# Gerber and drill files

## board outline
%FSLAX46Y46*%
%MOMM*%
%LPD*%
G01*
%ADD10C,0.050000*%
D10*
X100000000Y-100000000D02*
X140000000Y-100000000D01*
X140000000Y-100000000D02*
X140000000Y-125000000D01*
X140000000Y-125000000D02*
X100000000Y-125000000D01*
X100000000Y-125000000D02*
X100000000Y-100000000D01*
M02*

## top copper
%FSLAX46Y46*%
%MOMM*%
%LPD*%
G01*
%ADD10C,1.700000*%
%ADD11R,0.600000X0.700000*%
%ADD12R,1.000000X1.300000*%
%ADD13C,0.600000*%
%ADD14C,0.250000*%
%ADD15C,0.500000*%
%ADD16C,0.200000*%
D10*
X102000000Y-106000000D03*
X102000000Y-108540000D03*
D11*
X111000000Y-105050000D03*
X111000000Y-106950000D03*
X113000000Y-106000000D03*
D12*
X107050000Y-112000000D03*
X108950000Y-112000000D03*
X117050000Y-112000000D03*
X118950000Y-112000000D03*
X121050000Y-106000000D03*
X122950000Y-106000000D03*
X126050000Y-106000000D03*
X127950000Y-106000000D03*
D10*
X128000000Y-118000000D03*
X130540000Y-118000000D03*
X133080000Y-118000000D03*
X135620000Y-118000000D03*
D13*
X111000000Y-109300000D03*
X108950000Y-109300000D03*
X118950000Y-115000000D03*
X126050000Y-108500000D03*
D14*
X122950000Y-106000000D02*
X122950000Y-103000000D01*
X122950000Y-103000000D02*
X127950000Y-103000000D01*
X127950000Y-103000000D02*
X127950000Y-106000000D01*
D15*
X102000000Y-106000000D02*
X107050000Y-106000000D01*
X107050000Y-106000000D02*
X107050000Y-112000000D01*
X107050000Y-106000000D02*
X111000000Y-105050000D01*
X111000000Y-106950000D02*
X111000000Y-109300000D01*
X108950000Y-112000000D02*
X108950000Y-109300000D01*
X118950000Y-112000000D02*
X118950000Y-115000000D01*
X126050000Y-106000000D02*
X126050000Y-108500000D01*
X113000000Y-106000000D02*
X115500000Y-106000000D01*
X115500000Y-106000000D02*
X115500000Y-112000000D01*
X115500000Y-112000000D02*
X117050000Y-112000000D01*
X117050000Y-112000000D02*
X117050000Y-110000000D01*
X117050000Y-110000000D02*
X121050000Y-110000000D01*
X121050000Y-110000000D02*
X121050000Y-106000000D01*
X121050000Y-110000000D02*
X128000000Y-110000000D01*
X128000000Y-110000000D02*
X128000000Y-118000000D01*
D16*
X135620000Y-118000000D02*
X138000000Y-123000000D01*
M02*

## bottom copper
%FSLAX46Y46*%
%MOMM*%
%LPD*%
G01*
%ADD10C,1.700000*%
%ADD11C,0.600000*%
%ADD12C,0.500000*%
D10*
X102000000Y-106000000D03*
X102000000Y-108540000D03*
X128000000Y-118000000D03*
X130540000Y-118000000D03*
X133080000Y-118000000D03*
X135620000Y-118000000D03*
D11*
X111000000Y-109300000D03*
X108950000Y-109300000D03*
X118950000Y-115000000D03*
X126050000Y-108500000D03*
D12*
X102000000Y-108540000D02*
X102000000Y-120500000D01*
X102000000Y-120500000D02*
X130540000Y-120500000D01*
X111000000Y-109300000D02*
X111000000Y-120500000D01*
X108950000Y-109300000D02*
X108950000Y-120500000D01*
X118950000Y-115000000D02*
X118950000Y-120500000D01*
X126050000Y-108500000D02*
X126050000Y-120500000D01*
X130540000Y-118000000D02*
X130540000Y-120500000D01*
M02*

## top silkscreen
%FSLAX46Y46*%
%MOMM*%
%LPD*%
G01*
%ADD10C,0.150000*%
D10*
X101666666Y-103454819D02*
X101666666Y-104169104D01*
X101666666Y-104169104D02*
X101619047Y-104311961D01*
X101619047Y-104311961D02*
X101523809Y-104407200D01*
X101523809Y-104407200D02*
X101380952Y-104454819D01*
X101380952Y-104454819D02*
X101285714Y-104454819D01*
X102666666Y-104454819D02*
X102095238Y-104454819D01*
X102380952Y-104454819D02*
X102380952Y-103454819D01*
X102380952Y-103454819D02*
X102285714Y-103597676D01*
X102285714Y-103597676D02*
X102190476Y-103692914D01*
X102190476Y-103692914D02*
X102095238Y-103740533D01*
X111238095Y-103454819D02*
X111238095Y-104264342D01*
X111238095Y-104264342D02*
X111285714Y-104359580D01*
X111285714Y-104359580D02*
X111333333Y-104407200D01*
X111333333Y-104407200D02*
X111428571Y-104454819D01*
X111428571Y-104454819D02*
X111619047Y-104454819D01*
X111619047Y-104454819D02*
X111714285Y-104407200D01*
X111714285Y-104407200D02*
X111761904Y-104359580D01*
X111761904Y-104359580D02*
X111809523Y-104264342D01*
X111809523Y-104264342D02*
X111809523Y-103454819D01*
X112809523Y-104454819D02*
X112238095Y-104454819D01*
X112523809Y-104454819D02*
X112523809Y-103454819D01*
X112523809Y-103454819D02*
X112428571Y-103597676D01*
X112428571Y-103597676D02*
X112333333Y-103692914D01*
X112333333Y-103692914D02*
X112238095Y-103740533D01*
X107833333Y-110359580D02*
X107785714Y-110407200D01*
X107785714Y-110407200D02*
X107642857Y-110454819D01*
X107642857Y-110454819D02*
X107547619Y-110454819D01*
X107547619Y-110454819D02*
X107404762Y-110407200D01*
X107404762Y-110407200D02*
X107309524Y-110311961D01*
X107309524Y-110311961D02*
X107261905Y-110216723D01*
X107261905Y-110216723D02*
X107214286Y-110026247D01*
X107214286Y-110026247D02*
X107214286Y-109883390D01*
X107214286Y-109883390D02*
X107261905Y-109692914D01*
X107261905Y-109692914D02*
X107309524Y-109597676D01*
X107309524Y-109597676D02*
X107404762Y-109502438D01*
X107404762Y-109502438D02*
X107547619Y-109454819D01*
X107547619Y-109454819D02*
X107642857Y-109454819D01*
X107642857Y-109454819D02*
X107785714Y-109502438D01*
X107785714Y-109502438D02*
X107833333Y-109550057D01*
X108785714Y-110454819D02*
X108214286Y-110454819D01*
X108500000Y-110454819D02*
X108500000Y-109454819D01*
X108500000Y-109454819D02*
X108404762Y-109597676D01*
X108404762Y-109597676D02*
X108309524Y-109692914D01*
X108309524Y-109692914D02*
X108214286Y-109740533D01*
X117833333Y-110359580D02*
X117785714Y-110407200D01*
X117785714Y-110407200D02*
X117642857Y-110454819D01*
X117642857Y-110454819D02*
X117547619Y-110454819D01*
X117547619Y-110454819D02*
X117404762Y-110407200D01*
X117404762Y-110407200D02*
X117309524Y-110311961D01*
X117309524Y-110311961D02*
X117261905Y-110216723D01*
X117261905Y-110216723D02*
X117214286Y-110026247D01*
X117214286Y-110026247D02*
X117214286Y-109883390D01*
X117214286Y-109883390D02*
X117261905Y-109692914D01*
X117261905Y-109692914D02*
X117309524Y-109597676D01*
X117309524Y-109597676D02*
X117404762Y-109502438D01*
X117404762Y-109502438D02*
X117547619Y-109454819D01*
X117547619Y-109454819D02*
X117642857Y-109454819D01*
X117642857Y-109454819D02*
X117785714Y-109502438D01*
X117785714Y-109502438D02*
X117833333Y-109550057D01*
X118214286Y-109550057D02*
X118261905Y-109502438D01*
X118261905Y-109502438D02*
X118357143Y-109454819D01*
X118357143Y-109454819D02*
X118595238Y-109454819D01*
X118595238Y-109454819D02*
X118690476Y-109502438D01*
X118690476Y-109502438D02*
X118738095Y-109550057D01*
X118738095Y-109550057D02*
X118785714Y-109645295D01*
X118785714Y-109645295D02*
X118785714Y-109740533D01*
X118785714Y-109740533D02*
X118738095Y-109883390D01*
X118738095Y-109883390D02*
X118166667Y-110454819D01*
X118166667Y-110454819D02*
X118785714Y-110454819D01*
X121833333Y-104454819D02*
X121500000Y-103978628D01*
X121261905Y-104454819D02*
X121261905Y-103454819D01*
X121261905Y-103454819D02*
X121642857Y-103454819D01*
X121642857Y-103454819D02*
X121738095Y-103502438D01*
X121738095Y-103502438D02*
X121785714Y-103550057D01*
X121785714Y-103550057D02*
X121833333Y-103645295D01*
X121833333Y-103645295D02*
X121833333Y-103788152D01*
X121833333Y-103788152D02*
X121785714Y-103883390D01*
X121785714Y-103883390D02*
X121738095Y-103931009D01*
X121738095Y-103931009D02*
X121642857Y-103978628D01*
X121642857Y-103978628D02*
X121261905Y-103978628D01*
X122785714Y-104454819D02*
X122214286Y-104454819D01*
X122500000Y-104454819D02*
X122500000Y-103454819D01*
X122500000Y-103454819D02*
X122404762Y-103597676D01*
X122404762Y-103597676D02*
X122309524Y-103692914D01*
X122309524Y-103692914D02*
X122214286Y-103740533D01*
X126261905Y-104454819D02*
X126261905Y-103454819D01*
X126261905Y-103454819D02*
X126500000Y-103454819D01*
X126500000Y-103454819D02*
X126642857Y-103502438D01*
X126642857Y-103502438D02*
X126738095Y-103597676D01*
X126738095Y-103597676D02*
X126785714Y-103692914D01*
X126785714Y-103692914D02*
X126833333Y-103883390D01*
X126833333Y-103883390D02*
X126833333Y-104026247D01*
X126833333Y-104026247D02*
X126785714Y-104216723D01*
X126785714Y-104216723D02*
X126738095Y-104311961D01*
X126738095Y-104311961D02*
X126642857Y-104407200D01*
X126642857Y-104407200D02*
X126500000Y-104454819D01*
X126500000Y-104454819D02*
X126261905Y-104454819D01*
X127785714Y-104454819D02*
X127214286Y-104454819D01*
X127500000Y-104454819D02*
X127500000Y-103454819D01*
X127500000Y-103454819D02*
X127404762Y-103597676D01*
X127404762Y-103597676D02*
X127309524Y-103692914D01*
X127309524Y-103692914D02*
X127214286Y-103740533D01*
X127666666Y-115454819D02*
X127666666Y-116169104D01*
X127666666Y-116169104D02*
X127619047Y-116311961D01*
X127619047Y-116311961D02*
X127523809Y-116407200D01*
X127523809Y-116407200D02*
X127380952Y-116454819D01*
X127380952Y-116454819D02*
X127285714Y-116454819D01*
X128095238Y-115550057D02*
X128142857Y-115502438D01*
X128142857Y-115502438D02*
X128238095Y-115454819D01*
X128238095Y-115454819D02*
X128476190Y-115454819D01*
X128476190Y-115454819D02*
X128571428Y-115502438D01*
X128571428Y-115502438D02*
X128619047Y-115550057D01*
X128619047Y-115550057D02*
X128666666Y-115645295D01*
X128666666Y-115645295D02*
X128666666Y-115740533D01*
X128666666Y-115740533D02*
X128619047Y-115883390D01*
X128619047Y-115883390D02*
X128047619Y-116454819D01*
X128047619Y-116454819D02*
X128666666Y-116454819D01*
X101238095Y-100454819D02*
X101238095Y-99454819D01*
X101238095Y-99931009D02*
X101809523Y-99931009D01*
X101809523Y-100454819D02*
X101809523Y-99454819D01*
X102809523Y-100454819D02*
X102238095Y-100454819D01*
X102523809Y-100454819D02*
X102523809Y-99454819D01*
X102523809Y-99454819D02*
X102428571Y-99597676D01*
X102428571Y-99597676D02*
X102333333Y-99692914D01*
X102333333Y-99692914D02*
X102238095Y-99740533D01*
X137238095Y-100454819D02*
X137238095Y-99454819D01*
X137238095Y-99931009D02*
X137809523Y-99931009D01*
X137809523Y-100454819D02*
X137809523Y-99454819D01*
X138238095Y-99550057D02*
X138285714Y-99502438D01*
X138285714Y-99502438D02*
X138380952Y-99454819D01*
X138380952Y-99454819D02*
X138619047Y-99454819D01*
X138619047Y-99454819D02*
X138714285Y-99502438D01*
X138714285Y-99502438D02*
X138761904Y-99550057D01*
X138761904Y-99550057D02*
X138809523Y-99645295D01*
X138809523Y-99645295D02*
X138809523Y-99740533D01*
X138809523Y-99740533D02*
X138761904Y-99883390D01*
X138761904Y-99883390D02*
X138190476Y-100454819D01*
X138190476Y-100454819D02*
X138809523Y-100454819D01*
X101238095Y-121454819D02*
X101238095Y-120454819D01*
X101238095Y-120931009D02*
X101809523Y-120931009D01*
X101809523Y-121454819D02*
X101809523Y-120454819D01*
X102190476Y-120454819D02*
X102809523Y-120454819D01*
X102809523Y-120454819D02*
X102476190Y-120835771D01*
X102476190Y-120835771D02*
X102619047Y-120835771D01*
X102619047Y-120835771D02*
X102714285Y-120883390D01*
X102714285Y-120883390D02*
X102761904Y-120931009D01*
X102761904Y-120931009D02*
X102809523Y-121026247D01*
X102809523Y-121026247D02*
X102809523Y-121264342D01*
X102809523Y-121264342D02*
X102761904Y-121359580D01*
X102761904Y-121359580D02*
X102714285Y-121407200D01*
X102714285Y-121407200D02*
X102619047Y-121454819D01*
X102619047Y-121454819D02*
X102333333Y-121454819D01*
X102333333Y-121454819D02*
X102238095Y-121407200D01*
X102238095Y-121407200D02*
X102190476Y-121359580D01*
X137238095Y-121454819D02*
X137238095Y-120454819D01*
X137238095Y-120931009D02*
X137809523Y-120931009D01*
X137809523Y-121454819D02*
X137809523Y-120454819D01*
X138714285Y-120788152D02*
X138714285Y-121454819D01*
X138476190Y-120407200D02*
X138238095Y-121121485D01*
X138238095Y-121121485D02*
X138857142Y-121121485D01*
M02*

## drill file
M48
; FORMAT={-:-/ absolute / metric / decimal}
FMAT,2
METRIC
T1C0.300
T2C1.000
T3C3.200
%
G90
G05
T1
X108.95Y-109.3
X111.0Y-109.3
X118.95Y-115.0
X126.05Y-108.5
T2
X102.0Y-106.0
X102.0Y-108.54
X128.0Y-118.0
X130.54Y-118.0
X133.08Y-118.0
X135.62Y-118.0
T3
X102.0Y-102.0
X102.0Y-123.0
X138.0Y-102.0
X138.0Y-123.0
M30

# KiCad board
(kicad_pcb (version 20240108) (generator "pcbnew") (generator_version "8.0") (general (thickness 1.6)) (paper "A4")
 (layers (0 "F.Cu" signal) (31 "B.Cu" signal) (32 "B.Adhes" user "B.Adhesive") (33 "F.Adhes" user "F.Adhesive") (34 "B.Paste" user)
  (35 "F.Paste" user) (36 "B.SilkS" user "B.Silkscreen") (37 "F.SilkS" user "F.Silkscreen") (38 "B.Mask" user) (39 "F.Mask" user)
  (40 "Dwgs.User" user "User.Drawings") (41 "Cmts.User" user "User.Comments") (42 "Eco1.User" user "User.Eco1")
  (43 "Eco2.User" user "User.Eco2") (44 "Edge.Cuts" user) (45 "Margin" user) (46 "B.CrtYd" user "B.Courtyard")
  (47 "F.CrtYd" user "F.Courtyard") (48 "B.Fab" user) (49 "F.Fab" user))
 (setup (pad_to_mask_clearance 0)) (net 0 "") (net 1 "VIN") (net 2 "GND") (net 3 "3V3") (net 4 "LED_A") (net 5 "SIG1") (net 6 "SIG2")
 (gr_line (start 100 100) (end 140 100) (stroke (width 0.05) (type default)) (layer "Edge.Cuts"))
 (gr_line (start 140 100) (end 140 125) (stroke (width 0.05) (type default)) (layer "Edge.Cuts"))
 (gr_line (start 140 125) (end 100 125) (stroke (width 0.05) (type default)) (layer "Edge.Cuts"))
 (gr_line (start 100 125) (end 100 100) (stroke (width 0.05) (type default)) (layer "Edge.Cuts"))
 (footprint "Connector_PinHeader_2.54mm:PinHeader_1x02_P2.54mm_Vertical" (layer "F.Cu") (at 102 106)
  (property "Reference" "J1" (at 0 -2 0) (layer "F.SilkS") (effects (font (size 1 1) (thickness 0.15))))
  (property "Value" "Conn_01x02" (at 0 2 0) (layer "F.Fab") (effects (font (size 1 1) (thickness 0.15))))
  (pad "1" thru_hole circle (at 0 0) (size 1.7 1.7) (drill 1) (layers "*.Cu" "*.Mask") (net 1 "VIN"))
  (pad "2" thru_hole circle (at 0 2.54) (size 1.7 1.7) (drill 1) (layers "*.Cu" "*.Mask") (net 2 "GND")))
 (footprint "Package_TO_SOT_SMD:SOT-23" (layer "F.Cu") (at 112 106)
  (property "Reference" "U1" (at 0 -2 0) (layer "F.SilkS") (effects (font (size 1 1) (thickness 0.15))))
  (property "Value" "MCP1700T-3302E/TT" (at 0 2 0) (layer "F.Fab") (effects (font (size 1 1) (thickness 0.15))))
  (pad "1" smd rect (at -1 -0.95) (size 0.6 0.7) (layers "F.Cu" "F.Paste" "F.Mask") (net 1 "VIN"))
  (pad "2" smd rect (at -1 0.95) (size 0.6 0.7) (layers "F.Cu" "F.Paste" "F.Mask") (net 2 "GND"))
  (pad "3" smd rect (at 1 0) (size 0.6 0.7) (layers "F.Cu" "F.Paste" "F.Mask") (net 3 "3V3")))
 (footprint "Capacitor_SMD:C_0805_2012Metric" (layer "F.Cu") (at 108 112)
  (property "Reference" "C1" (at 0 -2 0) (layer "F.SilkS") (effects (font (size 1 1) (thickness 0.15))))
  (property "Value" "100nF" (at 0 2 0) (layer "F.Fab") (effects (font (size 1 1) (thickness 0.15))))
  (pad "1" smd rect (at -0.95 0) (size 1 1.3) (layers "F.Cu" "F.Paste" "F.Mask") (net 1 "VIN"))
  (pad "2" smd rect (at 0.95 0) (size 1 1.3) (layers "F.Cu" "F.Paste" "F.Mask") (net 2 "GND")))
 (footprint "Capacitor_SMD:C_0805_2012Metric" (layer "F.Cu") (at 118 112)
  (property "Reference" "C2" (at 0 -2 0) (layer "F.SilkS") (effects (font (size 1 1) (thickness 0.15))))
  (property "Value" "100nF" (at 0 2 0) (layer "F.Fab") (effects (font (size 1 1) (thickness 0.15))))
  (pad "1" smd rect (at -0.95 0) (size 1 1.3) (layers "F.Cu" "F.Paste" "F.Mask") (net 3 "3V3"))
  (pad "2" smd rect (at 0.95 0) (size 1 1.3) (layers "F.Cu" "F.Paste" "F.Mask") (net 2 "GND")))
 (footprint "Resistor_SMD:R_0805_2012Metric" (layer "F.Cu") (at 122 106)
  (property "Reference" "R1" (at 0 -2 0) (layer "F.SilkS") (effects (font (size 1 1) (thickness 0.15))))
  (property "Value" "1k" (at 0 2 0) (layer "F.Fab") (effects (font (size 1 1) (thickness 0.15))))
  (pad "1" smd rect (at -0.95 0) (size 1 1.3) (layers "F.Cu" "F.Paste" "F.Mask") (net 3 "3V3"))
  (pad "2" smd rect (at 0.95 0) (size 1 1.3) (layers "F.Cu" "F.Paste" "F.Mask") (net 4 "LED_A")))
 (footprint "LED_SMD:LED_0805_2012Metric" (layer "F.Cu") (at 127 106)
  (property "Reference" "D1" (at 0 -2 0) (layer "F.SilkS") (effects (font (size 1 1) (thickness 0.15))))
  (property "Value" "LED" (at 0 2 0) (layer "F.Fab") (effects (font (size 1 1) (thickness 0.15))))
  (pad "1" smd rect (at -0.95 0) (size 1 1.3) (layers "F.Cu" "F.Paste" "F.Mask") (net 2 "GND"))
  (pad "2" smd rect (at 0.95 0) (size 1 1.3) (layers "F.Cu" "F.Paste" "F.Mask") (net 4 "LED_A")))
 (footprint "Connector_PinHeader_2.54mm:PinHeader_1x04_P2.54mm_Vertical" (layer "F.Cu") (at 128 118)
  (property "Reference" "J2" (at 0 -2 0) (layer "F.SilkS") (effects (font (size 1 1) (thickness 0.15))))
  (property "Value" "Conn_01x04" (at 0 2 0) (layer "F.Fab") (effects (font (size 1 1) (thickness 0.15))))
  (pad "1" thru_hole circle (at 0 0) (size 1.7 1.7) (drill 1) (layers "*.Cu" "*.Mask") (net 3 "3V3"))
  (pad "2" thru_hole circle (at 2.54 0) (size 1.7 1.7) (drill 1) (layers "*.Cu" "*.Mask") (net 2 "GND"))
  (pad "3" thru_hole circle (at 5.08 0) (size 1.7 1.7) (drill 1) (layers "*.Cu" "*.Mask") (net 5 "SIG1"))
  (pad "4" thru_hole circle (at 7.62 0) (size 1.7 1.7) (drill 1) (layers "*.Cu" "*.Mask") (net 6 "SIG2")))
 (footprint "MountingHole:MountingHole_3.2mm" (layer "F.Cu") (at 102 102)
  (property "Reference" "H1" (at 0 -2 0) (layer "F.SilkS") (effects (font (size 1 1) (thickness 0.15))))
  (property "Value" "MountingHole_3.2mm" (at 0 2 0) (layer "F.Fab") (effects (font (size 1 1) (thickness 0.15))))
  (pad "1" np_thru_hole circle (at 0 0) (size 3.2 3.2) (drill 3.2) (layers "*.Cu" "*.Mask")))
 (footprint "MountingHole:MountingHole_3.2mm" (layer "F.Cu") (at 138 102)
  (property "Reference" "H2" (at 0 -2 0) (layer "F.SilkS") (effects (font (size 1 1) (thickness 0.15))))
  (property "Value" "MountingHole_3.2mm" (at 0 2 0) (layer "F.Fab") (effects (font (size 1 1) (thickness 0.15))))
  (pad "1" np_thru_hole circle (at 0 0) (size 3.2 3.2) (drill 3.2) (layers "*.Cu" "*.Mask")))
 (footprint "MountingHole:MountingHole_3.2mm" (layer "F.Cu") (at 102 123)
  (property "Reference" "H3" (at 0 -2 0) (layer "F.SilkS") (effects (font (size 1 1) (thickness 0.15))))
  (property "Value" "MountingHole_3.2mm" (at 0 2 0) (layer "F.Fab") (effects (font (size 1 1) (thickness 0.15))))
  (pad "1" np_thru_hole circle (at 0 0) (size 3.2 3.2) (drill 3.2) (layers "*.Cu" "*.Mask")))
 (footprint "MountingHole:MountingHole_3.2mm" (layer "F.Cu") (at 138 123)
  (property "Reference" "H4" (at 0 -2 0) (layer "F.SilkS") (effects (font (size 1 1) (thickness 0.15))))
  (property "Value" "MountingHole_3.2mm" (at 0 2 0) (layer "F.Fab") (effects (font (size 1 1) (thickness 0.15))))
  (pad "1" np_thru_hole circle (at 0 0) (size 3.2 3.2) (drill 3.2) (layers "*.Cu" "*.Mask")))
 (segment (start 122.95 106) (end 122.95 103) (width 0.25) (layer "F.Cu") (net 4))
 (segment (start 122.95 103) (end 127.95 103) (width 0.25) (layer "F.Cu") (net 4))
 (segment (start 127.95 103) (end 127.95 106) (width 0.25) (layer "F.Cu") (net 4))
 (segment (start 102 106) (end 107.05 106) (width 0.5) (layer "F.Cu") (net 1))
 (segment (start 107.05 106) (end 107.05 112) (width 0.5) (layer "F.Cu") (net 1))
 (segment (start 107.05 106) (end 111 105.05) (width 0.5) (layer "F.Cu") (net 1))
 (segment (start 111 106.95) (end 111 109.3) (width 0.5) (layer "F.Cu") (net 2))
 (segment (start 108.95 112) (end 108.95 109.3) (width 0.5) (layer "F.Cu") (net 2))
 (segment (start 118.95 112) (end 118.95 115) (width 0.5) (layer "F.Cu") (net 2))
 (segment (start 126.05 106) (end 126.05 108.5) (width 0.5) (layer "F.Cu") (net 2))
 (segment (start 113 106) (end 115.5 106) (width 0.5) (layer "F.Cu") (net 3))
 (segment (start 115.5 106) (end 115.5 112) (width 0.5) (layer "F.Cu") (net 3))
 (segment (start 115.5 112) (end 117.05 112) (width 0.5) (layer "F.Cu") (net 3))
 (segment (start 117.05 112) (end 117.05 110) (width 0.5) (layer "F.Cu") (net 3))
 (segment (start 117.05 110) (end 121.05 110) (width 0.5) (layer "F.Cu") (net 3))
 (segment (start 121.05 110) (end 121.05 106) (width 0.5) (layer "F.Cu") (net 3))
 (segment (start 121.05 110) (end 128 110) (width 0.5) (layer "F.Cu") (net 3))
 (segment (start 128 110) (end 128 118) (width 0.5) (layer "F.Cu") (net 3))
 (segment (start 102 108.54) (end 102 120.5) (width 0.5) (layer "B.Cu") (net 2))
 (segment (start 102 120.5) (end 130.54 120.5) (width 0.5) (layer "B.Cu") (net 2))
 (segment (start 111 109.3) (end 111 120.5) (width 0.5) (layer "B.Cu") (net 2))
 (segment (start 108.95 109.3) (end 108.95 120.5) (width 0.5) (layer "B.Cu") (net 2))
 (segment (start 118.95 115) (end 118.95 120.5) (width 0.5) (layer "B.Cu") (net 2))
 (segment (start 126.05 108.5) (end 126.05 120.5) (width 0.5) (layer "B.Cu") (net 2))
 (segment (start 130.54 118) (end 130.54 120.5) (width 0.5) (layer "B.Cu") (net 2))
 (via (at 111 109.3) (size 0.6) (drill 0.3) (layers "F.Cu" "B.Cu") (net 2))
 (via (at 108.95 109.3) (size 0.6) (drill 0.3) (layers "F.Cu" "B.Cu") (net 2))
 (via (at 118.95 115) (size 0.6) (drill 0.3) (layers "F.Cu" "B.Cu") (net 2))
 (via (at 126.05 108.5) (size 0.6) (drill 0.3) (layers "F.Cu" "B.Cu") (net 2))
 (segment (start 135.62 118) (end 138 123) (width 0.2) (layer "F.Cu") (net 6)))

